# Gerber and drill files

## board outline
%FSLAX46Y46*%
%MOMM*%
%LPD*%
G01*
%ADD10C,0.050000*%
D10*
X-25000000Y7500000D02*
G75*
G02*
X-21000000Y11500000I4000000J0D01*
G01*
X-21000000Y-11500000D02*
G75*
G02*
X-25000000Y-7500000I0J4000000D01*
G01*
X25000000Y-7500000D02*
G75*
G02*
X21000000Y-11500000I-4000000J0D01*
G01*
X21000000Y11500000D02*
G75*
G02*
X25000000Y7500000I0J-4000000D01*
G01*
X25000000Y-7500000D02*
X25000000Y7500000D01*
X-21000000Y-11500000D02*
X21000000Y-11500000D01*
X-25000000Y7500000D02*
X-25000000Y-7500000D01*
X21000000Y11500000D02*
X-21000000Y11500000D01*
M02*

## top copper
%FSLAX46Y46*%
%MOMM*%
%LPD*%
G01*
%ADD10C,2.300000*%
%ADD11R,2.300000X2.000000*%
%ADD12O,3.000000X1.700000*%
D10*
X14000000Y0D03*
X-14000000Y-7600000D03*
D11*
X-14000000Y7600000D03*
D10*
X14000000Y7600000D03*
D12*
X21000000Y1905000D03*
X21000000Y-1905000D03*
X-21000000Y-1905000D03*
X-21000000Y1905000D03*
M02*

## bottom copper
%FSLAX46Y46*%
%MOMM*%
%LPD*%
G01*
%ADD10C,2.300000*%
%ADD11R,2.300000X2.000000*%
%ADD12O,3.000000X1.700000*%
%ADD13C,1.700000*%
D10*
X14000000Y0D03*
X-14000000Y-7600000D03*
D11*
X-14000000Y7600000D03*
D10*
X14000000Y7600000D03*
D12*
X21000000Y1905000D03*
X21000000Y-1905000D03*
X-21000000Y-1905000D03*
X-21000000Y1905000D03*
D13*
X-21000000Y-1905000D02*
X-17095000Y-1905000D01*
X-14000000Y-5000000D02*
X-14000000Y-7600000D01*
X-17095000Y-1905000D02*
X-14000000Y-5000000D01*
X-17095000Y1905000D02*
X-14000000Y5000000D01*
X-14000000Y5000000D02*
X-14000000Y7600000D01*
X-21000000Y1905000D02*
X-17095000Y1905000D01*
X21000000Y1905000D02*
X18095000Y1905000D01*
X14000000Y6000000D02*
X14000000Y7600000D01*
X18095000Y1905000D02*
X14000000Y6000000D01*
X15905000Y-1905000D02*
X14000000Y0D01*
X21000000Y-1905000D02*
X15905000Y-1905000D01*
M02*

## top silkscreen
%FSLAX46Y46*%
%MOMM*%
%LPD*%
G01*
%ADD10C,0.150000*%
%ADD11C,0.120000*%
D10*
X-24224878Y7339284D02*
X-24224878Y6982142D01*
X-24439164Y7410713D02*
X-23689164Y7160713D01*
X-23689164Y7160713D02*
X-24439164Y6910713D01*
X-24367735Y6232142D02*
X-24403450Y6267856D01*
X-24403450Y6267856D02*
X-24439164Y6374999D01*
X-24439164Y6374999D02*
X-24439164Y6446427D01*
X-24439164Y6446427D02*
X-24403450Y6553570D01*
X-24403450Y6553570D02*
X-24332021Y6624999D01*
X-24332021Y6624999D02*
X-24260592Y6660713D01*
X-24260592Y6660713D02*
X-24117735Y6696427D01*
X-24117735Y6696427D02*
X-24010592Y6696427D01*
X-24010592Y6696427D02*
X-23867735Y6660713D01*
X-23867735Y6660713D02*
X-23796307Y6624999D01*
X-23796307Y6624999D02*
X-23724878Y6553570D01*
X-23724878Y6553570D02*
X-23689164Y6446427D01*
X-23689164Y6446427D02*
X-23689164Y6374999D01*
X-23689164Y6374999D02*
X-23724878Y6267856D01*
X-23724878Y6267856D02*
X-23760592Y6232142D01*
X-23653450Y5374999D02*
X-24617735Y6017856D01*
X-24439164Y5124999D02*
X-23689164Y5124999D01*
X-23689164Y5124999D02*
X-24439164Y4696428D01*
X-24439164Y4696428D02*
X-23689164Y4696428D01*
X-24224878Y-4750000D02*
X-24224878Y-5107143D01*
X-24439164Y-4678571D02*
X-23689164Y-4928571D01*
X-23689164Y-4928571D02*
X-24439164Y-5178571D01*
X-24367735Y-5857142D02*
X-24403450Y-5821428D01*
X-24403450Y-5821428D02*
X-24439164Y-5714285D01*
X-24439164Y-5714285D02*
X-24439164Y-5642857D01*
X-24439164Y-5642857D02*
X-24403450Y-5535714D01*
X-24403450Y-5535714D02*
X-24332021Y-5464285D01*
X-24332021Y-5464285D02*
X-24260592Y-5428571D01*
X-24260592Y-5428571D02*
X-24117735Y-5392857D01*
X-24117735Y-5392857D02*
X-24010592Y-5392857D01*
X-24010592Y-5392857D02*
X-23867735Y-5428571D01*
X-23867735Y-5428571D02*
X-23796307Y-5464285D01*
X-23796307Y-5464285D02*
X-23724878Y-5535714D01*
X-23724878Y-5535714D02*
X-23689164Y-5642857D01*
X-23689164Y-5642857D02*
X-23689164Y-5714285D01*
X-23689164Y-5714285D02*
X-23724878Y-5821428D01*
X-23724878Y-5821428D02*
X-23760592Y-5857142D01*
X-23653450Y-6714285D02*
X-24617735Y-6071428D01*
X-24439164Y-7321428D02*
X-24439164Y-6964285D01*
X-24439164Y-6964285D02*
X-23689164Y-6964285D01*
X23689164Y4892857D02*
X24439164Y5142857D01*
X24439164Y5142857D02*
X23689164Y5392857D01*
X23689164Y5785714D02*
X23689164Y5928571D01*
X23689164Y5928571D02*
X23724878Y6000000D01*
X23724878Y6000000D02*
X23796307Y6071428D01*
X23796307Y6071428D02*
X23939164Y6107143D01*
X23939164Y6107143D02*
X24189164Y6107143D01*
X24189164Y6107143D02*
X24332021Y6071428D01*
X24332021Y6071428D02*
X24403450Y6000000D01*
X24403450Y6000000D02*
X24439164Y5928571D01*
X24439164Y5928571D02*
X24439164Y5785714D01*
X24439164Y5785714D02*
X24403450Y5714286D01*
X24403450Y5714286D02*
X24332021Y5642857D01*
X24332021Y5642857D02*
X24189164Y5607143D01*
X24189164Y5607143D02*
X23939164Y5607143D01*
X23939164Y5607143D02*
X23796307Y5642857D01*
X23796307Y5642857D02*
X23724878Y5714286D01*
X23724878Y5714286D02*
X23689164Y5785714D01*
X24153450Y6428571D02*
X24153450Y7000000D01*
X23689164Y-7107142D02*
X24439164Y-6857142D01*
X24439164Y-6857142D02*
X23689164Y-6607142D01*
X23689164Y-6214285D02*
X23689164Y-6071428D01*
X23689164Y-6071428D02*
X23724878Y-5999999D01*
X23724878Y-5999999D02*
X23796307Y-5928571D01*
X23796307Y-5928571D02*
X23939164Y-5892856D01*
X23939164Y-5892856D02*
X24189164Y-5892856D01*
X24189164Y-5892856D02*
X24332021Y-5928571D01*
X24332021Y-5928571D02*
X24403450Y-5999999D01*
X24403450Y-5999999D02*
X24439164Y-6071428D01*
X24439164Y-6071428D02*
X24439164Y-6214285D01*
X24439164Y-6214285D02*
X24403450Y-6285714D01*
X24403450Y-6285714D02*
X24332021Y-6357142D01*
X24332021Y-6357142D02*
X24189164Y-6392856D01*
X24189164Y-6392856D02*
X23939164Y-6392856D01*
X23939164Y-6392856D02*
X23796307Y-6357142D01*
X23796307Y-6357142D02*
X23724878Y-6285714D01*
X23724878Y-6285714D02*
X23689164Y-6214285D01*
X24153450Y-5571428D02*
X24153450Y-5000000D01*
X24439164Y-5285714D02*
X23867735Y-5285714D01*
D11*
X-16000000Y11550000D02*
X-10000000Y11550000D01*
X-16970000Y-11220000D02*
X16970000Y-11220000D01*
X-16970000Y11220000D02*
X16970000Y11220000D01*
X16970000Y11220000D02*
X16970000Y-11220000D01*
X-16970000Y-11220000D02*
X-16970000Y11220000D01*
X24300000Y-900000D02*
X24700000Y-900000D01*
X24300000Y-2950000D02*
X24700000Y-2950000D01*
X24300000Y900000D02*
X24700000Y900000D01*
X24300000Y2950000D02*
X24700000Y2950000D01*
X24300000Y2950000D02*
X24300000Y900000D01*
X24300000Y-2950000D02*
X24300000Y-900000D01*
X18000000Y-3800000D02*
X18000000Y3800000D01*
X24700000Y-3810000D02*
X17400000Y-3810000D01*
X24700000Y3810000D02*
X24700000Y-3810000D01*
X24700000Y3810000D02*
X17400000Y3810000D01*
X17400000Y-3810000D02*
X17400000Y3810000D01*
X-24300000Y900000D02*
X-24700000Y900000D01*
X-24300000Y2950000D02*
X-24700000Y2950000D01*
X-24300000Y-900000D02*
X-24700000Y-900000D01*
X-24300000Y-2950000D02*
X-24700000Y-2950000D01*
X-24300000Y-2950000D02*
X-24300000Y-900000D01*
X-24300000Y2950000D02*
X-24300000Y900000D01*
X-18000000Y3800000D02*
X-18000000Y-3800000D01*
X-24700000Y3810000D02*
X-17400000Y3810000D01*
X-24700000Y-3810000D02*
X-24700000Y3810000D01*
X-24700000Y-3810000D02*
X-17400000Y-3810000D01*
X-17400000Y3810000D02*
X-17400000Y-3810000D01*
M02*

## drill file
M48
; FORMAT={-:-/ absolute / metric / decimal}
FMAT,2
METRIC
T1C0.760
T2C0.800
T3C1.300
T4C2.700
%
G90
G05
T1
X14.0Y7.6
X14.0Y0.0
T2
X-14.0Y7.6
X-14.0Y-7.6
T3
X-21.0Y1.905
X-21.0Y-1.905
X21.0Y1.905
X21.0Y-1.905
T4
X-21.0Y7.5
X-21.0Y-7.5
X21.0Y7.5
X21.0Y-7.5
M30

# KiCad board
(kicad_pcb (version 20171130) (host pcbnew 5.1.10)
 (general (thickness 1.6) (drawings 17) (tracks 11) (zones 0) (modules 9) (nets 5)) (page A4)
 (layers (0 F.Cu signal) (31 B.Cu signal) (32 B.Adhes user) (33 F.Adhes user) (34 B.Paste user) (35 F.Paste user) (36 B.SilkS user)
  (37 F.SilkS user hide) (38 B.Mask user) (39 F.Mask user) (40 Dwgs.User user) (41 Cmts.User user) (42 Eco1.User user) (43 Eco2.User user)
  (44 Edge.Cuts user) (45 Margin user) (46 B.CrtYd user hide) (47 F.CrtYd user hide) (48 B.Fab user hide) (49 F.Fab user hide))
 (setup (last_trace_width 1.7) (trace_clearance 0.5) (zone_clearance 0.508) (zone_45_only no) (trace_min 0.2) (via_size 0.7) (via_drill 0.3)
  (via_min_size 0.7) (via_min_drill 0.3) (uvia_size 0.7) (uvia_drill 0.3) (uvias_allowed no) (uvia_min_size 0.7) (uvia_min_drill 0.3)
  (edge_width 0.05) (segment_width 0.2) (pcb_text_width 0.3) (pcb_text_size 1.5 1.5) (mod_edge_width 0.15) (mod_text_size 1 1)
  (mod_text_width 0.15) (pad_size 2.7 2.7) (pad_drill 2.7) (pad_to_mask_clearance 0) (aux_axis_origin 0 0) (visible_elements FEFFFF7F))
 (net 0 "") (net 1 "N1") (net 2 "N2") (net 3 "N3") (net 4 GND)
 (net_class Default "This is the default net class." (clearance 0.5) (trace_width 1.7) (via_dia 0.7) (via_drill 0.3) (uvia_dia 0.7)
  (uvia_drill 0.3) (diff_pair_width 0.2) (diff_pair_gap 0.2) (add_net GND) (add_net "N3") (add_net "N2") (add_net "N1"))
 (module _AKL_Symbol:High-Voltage (layer B.Cu) (at -13 0 90)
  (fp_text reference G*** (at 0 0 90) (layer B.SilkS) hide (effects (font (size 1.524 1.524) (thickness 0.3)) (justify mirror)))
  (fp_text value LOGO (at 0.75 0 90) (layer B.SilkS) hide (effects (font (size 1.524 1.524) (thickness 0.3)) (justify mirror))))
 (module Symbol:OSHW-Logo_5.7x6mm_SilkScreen (layer B.Cu) (at 13 7 90)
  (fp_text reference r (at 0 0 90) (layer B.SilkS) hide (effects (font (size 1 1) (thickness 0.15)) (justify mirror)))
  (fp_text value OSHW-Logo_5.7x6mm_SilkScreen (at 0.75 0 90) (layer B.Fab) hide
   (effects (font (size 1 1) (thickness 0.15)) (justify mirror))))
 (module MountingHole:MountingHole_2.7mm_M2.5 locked (layer F.Cu) (at 21 7.5)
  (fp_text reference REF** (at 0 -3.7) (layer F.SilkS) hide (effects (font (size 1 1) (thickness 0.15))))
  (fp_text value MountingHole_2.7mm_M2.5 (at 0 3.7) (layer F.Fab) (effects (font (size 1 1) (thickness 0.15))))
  (pad 1 np_thru_hole circle (at 0 0) (size 2.7 2.7) (drill 2.7) (layers *.Cu *.Mask)))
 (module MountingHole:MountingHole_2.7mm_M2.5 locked (layer F.Cu) (at 21 -7.5)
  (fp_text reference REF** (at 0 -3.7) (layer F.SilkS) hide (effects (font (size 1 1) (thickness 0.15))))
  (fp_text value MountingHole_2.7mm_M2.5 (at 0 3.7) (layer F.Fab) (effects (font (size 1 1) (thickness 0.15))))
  (pad 1 np_thru_hole circle (at 0 0) (size 2.7 2.7) (drill 2.7) (layers *.Cu *.Mask)))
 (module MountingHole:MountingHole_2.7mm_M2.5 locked (layer F.Cu) (at -21 7.5)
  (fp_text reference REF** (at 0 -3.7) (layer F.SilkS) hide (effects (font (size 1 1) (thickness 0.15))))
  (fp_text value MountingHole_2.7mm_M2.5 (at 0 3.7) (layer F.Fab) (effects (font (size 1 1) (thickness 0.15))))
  (pad 1 np_thru_hole circle (at 0 0) (size 2.7 2.7) (drill 2.7) (layers *.Cu *.Mask)))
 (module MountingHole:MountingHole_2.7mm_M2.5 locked (layer F.Cu) (at -21 -7.5)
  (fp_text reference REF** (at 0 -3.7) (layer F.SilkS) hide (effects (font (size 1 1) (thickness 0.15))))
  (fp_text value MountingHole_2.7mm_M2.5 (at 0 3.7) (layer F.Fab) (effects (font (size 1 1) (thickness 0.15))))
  (pad 1 np_thru_hole circle (at 0 0) (size 2.7 2.7) (drill 2.7) (layers *.Cu *.Mask)))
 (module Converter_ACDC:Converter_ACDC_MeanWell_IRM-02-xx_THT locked (layer F.Cu) (at -14 -7.6)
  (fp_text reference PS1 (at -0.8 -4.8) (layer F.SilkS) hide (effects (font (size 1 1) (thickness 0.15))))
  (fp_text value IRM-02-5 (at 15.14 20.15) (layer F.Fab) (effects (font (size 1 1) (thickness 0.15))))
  (fp_line (start -2 -3.95) (end 4 -3.95) (layer F.SilkS) (width 0.12))
  (fp_line (start -2.97 18.82) (end 30.97 18.82) (layer F.SilkS) (width 0.12))
  (fp_line (start -2.97 -3.62) (end 30.97 -3.62) (layer F.SilkS) (width 0.12))
  (fp_line (start 30.97 -3.62) (end 30.97 18.82) (layer F.SilkS) (width 0.12))
  (fp_line (start -2.97 18.82) (end -2.97 -3.62) (layer F.SilkS) (width 0.12))
  (pad 4 thru_hole circle (at 28 7.6) (size 2.3 2.3) (drill 0.76) (layers *.Cu *.Mask) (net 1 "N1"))
  (pad 2 thru_hole circle (at 0 15.2) (size 2.3 2.3) (drill 0.8) (layers *.Cu *.Mask) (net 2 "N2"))
  (pad 1 thru_hole rect (at 0 0) (size 2.3 2) (drill 0.8) (layers *.Cu *.Mask) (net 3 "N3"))
  (pad 3 thru_hole circle (at 28 0) (size 2.3 2.3) (drill 0.76) (layers *.Cu *.Mask) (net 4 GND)))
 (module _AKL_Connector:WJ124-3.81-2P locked (layer F.Cu) (at 21 0 90)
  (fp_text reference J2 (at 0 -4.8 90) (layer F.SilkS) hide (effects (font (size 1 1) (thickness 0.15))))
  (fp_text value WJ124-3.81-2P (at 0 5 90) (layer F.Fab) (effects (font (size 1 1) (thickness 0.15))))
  (fp_line (start -0.9 3.3) (end -0.9 3.7) (layer F.SilkS) (width 0.12))
  (fp_line (start -2.95 3.3) (end -2.95 3.7) (layer F.SilkS) (width 0.12))
  (fp_line (start 0.9 3.3) (end 0.9 3.7) (layer F.SilkS) (width 0.12))
  (fp_line (start 2.95 3.3) (end 2.95 3.7) (layer F.SilkS) (width 0.12))
  (fp_line (start 2.95 3.3) (end 0.9 3.3) (layer F.SilkS) (width 0.12))
  (fp_line (start -2.95 3.3) (end -0.9 3.3) (layer F.SilkS) (width 0.12))
  (fp_line (start -3.8 -3) (end 3.8 -3) (layer F.SilkS) (width 0.12))
  (fp_line (start -3.81 3.7) (end -3.81 -3.6) (layer F.SilkS) (width 0.12))
  (fp_line (start 3.81 3.7) (end -3.81 3.7) (layer F.SilkS) (width 0.12))
  (fp_line (start 3.81 3.7) (end 3.81 -3.6) (layer F.SilkS) (width 0.12))
  (fp_line (start -3.81 -3.6) (end 3.81 -3.6) (layer F.SilkS) (width 0.12))
  (pad 2 thru_hole oval (at 1.905 0 180) (size 3 1.7) (drill 1.3) (layers *.Cu *.Mask) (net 4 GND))
  (pad 1 thru_hole oval (at -1.905 0 180) (size 3 1.7) (drill 1.3) (layers *.Cu *.Mask) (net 1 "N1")))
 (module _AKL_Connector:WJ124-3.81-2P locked (layer F.Cu) (at -21 0 270)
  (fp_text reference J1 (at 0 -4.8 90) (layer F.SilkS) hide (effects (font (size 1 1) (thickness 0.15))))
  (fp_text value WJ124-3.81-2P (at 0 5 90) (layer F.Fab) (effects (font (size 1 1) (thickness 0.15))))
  (fp_line (start -0.9 3.3) (end -0.9 3.7) (layer F.SilkS) (width 0.12))
  (fp_line (start -2.95 3.3) (end -2.95 3.7) (layer F.SilkS) (width 0.12))
  (fp_line (start 0.9 3.3) (end 0.9 3.7) (layer F.SilkS) (width 0.12))
  (fp_line (start 2.95 3.3) (end 2.95 3.7) (layer F.SilkS) (width 0.12))
  (fp_line (start 2.95 3.3) (end 0.9 3.3) (layer F.SilkS) (width 0.12))
  (fp_line (start -2.95 3.3) (end -0.9 3.3) (layer F.SilkS) (width 0.12))
  (fp_line (start -3.8 -3) (end 3.8 -3) (layer F.SilkS) (width 0.12))
  (fp_line (start -3.81 3.7) (end -3.81 -3.6) (layer F.SilkS) (width 0.12))
  (fp_line (start 3.81 3.7) (end -3.81 3.7) (layer F.SilkS) (width 0.12))
  (fp_line (start 3.81 3.7) (end 3.81 -3.6) (layer F.SilkS) (width 0.12))
  (fp_line (start -3.81 -3.6) (end 3.81 -3.6) (layer F.SilkS) (width 0.12))
  (pad 2 thru_hole oval (at 1.905 0) (size 3 1.7) (drill 1.3) (layers *.Cu *.Mask) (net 2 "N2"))
  (pad 1 thru_hole oval (at -1.905 0) (size 3 1.7) (drill 1.3) (layers *.Cu *.Mask) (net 3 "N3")))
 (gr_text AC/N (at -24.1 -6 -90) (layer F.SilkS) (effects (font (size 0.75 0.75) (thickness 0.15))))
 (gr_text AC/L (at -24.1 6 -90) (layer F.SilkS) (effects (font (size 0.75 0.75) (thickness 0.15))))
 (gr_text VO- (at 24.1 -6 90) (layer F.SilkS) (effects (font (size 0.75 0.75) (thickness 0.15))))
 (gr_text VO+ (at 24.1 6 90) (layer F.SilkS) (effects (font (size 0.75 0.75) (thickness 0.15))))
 (gr_arc (start -21 -7.5) (end -21 -11.5) (angle -90) (layer Edge.Cuts) (width 0.05))
 (gr_arc (start -21 7.5) (end -25 7.5) (angle -90) (layer Edge.Cuts) (width 0.05))
 (gr_arc (start 21 7.5) (end 21 11.5) (angle -90) (layer Edge.Cuts) (width 0.05))
 (gr_arc (start 21 -7.5) (end 25 -7.5) (angle -90) (layer Edge.Cuts) (width 0.05))
 (gr_line (start 25 7.5) (end 25 -7.5) (layer Edge.Cuts) (width 0.05))
 (gr_line (start -21 11.5) (end 21 11.5) (layer Edge.Cuts) (width 0.05))
 (gr_line (start -25 -7.5) (end -25 7.5) (layer Edge.Cuts) (width 0.05))
 (gr_line (start 21 -11.5) (end -21 -11.5) (layer Edge.Cuts) (width 0.05))
 (segment (start -21 1.905) (end -17.095 1.905) (width 1.7) (layer B.Cu) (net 2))
 (segment (start -14 5) (end -14 7.6) (width 1.7) (layer B.Cu) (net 2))
 (segment (start -17.095 1.905) (end -14 5) (width 1.7) (layer B.Cu) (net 2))
 (segment (start -17.095 -1.905) (end -14 -5) (width 1.7) (layer B.Cu) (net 3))
 (segment (start -14 -5) (end -14 -7.6) (width 1.7) (layer B.Cu) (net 3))
 (segment (start -21 -1.905) (end -17.095 -1.905) (width 1.7) (layer B.Cu) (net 3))
 (segment (start 21 -1.905) (end 18.095 -1.905) (width 1.7) (layer B.Cu) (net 4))
 (segment (start 14 -6) (end 14 -7.6) (width 1.7) (layer B.Cu) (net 4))
 (segment (start 18.095 -1.905) (end 14 -6) (width 1.7) (layer B.Cu) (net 4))
 (segment (start 15.905 1.905) (end 14 0) (width 1.7) (layer B.Cu) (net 1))
 (segment (start 21 1.905) (end 15.905 1.905) (width 1.7) (layer B.Cu) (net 1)))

